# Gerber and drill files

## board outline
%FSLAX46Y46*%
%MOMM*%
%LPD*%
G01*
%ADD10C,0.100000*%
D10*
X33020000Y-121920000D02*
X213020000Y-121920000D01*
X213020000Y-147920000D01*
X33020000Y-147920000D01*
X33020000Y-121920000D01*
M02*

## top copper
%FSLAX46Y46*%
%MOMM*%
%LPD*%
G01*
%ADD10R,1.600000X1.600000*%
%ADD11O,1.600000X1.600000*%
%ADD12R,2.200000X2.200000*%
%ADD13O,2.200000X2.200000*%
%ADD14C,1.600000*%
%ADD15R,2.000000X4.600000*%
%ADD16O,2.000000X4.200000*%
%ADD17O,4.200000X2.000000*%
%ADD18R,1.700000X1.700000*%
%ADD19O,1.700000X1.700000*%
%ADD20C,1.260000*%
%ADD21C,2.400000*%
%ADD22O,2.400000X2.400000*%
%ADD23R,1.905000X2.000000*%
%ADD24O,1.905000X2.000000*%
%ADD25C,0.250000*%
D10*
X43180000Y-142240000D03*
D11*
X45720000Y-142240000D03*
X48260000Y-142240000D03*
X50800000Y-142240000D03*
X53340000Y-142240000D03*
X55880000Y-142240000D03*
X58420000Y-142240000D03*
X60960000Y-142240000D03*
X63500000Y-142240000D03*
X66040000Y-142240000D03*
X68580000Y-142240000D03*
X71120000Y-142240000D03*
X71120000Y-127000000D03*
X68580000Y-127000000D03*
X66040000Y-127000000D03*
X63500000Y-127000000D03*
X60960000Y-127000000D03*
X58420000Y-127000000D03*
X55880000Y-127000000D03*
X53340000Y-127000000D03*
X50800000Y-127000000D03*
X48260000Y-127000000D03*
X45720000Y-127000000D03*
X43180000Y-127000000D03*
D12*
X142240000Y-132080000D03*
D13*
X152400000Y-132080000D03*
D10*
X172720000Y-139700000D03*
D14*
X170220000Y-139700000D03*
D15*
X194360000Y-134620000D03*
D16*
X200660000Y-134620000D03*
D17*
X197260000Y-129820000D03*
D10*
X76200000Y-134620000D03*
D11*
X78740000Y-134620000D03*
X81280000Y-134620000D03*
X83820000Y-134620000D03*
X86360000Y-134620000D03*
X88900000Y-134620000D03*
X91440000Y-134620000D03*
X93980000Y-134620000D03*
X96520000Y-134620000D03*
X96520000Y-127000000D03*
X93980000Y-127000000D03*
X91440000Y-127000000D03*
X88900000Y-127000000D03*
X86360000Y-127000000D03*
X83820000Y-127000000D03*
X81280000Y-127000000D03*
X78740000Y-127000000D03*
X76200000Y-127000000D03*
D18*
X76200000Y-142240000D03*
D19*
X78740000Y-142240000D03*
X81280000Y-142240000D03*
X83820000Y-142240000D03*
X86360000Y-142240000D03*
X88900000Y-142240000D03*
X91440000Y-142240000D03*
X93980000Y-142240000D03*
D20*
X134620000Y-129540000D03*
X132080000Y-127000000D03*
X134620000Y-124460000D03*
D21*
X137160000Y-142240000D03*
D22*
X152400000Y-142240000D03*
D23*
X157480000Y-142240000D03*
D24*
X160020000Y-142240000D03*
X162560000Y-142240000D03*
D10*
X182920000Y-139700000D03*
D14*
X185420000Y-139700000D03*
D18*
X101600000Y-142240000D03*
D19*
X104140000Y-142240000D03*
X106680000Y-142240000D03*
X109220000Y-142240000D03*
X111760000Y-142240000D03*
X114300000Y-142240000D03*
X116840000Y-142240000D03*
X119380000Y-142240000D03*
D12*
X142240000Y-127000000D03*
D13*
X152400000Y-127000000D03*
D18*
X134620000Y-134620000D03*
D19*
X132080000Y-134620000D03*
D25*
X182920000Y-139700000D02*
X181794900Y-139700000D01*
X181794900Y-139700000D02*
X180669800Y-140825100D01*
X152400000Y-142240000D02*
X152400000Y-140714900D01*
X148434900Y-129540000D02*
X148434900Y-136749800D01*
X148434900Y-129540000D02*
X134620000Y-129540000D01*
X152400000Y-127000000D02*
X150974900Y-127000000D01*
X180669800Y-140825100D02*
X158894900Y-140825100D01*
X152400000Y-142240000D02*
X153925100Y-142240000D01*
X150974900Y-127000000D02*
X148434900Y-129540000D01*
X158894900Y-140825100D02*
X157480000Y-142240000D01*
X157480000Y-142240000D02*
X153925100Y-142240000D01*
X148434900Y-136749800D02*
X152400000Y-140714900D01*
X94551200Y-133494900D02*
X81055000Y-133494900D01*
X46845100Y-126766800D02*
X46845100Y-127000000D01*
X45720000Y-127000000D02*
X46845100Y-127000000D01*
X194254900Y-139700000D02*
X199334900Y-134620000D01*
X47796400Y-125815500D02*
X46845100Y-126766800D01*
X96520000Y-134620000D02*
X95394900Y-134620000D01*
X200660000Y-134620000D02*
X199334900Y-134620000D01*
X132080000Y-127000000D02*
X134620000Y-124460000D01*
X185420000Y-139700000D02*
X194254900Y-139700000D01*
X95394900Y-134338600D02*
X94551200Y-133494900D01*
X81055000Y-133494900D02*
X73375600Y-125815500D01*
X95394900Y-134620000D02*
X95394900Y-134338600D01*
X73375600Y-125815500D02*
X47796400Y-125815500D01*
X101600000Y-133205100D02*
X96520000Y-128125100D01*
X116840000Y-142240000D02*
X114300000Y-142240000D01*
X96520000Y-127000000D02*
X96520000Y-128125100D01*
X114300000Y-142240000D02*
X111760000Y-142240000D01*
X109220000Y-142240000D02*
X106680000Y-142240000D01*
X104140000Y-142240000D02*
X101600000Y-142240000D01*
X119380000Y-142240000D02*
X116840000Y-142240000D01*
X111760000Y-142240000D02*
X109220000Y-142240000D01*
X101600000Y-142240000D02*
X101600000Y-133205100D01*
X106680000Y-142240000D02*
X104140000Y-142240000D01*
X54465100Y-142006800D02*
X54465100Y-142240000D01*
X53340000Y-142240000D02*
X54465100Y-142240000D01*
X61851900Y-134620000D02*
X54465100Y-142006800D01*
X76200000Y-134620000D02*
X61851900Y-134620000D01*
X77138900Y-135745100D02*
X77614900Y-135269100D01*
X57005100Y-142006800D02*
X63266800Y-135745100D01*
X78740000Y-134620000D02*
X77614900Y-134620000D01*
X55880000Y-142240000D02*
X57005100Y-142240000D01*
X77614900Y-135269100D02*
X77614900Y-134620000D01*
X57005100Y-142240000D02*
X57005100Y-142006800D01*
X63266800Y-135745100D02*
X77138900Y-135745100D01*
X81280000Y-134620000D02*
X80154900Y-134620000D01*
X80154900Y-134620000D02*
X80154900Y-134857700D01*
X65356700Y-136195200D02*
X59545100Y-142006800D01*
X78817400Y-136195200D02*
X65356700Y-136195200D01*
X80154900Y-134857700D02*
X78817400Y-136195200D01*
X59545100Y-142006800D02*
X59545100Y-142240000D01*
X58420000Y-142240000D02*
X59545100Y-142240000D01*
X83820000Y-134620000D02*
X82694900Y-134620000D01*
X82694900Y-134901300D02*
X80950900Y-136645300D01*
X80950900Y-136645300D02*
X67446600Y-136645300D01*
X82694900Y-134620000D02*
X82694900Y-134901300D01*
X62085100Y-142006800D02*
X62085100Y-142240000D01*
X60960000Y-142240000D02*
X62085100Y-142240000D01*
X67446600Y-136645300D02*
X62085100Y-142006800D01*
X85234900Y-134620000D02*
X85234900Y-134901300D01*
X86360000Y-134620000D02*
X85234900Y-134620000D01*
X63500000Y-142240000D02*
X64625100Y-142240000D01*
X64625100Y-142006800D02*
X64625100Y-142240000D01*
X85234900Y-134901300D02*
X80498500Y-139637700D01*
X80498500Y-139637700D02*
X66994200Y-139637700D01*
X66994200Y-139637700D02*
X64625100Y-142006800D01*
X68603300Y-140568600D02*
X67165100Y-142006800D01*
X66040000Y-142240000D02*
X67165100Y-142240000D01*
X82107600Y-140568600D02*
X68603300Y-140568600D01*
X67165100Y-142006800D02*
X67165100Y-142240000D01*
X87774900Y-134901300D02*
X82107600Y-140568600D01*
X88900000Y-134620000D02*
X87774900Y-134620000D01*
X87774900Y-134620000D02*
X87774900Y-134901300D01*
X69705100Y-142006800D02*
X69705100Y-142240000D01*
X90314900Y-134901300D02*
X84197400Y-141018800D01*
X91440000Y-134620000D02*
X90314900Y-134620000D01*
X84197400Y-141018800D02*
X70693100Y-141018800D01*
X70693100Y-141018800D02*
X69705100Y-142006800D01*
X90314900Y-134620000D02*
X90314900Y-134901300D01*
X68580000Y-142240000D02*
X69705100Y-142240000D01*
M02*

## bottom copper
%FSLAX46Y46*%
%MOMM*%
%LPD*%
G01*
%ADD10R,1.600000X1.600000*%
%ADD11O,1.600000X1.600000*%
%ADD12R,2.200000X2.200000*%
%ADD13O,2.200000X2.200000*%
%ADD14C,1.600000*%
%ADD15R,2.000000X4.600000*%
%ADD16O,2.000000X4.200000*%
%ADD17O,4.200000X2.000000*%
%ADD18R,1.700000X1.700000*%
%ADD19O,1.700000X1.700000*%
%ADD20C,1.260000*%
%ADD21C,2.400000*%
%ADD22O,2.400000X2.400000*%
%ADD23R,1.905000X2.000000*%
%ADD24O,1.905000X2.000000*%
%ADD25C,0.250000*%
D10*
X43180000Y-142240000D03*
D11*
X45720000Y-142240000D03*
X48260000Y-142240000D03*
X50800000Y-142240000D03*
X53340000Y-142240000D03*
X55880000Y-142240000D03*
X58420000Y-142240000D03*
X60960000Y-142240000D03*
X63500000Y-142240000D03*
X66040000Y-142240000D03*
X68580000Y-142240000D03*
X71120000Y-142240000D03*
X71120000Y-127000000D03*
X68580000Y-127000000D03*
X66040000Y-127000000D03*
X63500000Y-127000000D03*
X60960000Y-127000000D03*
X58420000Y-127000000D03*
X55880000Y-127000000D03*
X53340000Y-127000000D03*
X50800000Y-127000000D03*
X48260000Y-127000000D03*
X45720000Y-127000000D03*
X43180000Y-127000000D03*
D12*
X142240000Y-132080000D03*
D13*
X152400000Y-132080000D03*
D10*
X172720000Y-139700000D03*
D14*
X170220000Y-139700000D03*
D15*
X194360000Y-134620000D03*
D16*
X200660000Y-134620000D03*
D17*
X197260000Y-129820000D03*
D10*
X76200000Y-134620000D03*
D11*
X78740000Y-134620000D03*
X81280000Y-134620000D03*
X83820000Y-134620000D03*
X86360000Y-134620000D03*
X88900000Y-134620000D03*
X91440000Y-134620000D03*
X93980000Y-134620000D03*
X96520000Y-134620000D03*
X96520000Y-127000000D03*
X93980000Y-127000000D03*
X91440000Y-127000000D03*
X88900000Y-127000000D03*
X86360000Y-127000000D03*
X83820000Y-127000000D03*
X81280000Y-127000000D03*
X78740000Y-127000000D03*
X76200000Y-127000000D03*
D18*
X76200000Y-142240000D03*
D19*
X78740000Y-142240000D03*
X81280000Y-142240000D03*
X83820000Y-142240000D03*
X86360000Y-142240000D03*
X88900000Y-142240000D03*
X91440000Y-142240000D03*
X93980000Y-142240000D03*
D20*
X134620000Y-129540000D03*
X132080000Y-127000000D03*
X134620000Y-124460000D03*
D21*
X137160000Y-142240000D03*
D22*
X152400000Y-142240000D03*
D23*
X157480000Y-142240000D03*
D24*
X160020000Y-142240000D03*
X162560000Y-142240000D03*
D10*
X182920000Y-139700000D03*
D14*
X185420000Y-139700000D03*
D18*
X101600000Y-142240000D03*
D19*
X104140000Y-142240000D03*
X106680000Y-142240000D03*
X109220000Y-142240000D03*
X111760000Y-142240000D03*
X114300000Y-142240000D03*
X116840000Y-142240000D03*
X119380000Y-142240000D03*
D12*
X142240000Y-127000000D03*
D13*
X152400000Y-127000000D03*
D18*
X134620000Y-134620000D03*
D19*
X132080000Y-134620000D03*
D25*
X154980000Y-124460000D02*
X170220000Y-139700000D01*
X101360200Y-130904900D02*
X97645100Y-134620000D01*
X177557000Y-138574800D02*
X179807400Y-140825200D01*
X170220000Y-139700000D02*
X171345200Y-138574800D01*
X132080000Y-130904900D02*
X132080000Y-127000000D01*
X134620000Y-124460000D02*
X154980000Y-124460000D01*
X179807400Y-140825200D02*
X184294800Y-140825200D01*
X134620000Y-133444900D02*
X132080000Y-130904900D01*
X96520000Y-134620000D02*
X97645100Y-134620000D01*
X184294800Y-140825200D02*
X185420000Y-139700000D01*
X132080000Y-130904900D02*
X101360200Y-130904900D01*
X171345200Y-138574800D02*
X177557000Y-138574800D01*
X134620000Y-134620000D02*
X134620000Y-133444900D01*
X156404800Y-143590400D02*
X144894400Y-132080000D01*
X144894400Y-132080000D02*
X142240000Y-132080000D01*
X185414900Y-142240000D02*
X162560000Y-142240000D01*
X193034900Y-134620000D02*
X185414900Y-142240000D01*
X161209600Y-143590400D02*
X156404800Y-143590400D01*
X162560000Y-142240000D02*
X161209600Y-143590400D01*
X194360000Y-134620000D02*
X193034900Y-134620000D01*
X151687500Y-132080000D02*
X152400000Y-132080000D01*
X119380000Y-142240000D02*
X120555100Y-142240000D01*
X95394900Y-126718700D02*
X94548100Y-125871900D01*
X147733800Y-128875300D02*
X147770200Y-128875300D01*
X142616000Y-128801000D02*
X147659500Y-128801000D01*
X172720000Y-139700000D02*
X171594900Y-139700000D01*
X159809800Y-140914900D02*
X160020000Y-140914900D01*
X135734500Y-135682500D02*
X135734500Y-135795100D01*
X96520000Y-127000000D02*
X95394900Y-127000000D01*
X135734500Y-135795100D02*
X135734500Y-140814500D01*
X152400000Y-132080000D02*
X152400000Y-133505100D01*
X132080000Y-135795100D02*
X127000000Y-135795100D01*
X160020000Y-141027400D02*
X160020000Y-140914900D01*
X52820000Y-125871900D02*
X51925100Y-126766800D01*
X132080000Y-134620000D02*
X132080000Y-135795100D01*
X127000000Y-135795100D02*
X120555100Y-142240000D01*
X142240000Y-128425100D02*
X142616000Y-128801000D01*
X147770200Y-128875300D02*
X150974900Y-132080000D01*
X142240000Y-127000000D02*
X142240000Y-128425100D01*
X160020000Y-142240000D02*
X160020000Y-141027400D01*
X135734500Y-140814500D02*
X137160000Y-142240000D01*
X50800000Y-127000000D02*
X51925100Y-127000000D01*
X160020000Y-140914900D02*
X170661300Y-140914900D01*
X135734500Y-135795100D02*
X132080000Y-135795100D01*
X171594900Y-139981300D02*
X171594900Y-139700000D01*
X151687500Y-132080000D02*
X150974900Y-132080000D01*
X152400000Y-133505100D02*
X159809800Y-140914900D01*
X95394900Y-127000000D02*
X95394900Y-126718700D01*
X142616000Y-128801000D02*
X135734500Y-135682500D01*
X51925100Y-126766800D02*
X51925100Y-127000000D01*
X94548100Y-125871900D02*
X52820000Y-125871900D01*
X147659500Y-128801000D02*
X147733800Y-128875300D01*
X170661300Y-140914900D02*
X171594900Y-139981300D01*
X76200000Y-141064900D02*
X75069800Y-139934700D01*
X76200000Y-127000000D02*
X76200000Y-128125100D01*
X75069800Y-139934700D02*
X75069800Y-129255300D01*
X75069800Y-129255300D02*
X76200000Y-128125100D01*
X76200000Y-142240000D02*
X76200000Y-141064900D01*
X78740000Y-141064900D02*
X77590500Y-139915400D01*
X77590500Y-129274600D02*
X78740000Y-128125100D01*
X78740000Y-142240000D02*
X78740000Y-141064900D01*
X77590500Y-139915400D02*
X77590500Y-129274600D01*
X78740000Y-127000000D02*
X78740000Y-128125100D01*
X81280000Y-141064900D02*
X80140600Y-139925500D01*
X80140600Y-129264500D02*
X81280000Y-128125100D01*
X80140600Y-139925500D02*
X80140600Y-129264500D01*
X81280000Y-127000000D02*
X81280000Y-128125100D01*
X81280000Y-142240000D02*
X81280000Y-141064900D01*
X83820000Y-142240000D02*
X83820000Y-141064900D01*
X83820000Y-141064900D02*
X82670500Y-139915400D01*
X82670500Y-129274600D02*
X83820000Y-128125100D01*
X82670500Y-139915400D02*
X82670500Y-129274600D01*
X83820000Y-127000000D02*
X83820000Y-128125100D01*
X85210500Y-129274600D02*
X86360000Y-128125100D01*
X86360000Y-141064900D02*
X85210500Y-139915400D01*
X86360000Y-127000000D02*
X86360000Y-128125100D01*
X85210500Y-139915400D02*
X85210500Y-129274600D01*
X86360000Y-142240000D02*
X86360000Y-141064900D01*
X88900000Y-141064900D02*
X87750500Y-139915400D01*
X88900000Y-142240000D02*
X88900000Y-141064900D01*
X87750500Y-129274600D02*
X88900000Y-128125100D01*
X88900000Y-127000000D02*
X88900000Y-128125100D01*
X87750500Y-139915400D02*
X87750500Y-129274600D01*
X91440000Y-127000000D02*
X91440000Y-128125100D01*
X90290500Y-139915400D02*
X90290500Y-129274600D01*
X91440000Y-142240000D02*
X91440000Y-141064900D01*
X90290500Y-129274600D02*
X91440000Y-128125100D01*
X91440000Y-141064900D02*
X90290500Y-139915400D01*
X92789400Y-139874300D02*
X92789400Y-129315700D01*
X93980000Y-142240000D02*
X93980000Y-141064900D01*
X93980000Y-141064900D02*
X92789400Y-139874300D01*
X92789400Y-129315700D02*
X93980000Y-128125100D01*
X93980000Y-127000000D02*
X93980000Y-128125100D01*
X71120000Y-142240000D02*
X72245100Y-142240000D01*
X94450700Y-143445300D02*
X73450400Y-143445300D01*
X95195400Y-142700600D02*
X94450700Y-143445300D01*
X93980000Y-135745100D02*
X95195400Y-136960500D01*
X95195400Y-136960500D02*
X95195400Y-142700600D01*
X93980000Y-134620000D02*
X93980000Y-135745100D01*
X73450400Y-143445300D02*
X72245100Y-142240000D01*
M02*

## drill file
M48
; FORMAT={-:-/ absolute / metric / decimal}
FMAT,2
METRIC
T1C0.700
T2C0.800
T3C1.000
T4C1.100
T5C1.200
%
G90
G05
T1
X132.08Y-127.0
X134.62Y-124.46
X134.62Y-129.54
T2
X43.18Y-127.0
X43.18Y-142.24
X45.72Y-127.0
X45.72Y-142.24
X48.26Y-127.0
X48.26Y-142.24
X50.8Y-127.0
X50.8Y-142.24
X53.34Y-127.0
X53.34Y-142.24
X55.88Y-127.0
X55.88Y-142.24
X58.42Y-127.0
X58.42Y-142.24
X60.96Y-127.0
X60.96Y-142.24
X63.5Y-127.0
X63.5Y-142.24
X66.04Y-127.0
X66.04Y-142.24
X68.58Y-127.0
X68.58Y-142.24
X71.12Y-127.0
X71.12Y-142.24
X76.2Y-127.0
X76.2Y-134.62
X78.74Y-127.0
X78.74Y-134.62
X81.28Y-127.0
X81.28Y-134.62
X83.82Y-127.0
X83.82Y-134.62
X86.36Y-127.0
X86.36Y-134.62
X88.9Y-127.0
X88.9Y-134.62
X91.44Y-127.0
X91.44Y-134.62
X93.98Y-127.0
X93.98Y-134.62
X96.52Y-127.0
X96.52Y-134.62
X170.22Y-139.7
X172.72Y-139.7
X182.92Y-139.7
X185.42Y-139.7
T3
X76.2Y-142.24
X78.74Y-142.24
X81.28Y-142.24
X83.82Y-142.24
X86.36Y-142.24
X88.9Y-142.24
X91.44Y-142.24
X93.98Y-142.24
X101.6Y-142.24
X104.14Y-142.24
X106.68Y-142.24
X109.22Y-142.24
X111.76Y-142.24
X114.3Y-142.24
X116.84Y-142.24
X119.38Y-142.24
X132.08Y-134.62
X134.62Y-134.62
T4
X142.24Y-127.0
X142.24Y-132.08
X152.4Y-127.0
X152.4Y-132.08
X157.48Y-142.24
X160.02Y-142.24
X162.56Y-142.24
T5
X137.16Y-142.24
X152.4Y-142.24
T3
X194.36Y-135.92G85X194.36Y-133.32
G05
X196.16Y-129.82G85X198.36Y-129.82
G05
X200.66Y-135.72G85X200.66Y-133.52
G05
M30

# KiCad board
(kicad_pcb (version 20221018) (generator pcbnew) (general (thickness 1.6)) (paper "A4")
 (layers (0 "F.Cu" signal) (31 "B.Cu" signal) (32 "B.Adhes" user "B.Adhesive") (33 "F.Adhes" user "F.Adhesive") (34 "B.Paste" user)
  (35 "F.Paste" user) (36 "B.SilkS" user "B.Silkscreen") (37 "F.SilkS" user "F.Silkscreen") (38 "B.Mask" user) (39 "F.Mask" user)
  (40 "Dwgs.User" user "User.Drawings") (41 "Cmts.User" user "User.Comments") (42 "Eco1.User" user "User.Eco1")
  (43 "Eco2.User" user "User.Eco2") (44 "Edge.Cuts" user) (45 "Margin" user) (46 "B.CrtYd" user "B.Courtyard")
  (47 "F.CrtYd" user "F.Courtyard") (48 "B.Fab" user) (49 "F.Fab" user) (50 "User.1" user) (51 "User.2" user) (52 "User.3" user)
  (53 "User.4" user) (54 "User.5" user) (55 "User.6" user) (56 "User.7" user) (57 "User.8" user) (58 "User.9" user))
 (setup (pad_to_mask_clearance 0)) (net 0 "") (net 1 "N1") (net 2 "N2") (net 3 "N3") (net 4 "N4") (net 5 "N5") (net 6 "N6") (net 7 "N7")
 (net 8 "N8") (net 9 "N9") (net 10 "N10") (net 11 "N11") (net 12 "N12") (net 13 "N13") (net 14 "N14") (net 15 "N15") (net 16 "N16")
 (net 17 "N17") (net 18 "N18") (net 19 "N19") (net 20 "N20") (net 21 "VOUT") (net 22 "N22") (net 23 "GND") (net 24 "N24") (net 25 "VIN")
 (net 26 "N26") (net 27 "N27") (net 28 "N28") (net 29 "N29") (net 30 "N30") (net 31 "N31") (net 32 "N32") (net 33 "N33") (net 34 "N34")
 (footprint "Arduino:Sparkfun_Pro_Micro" (layer "F.Cu") (at 71.12 127 -90)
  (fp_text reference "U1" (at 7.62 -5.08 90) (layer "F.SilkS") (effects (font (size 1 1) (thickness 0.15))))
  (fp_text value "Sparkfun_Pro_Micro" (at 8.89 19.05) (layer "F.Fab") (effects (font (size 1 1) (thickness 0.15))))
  (pad "1" thru_hole rect (at 15.24 27.94 270) (size 1.6 1.6) (drill 0.8) (layers "*.Cu" "*.Mask") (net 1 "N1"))
  (pad "2" thru_hole oval (at 15.24 25.4 270) (size 1.6 1.6) (drill 0.8) (layers "*.Cu" "*.Mask") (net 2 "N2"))
  (pad "3" thru_hole oval (at 15.24 22.86 270) (size 1.6 1.6) (drill 0.8) (layers "*.Cu" "*.Mask") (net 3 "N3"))
  (pad "4" thru_hole oval (at 15.24 20.32 270) (size 1.6 1.6) (drill 0.8) (layers "*.Cu" "*.Mask") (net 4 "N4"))
  (pad "5" thru_hole oval (at 15.24 17.78 270) (size 1.6 1.6) (drill 0.8) (layers "*.Cu" "*.Mask") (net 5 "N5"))
  (pad "6" thru_hole oval (at 15.24 15.24 270) (size 1.6 1.6) (drill 0.8) (layers "*.Cu" "*.Mask") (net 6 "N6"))
  (pad "7" thru_hole oval (at 15.24 12.7 270) (size 1.6 1.6) (drill 0.8) (layers "*.Cu" "*.Mask") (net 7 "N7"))
  (pad "8" thru_hole oval (at 15.24 10.16 270) (size 1.6 1.6) (drill 0.8) (layers "*.Cu" "*.Mask") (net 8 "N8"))
  (pad "9" thru_hole oval (at 15.24 7.62 270) (size 1.6 1.6) (drill 0.8) (layers "*.Cu" "*.Mask") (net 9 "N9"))
  (pad "10" thru_hole oval (at 15.24 5.08 270) (size 1.6 1.6) (drill 0.8) (layers "*.Cu" "*.Mask") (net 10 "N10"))
  (pad "11" thru_hole oval (at 15.24 2.54 270) (size 1.6 1.6) (drill 0.8) (layers "*.Cu" "*.Mask") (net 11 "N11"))
  (pad "12" thru_hole oval (at 15.24 0 270) (size 1.6 1.6) (drill 0.8) (layers "*.Cu" "*.Mask") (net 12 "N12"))
  (pad "13" thru_hole oval (at 0 0 270) (size 1.6 1.6) (drill 0.8) (layers "*.Cu" "*.Mask") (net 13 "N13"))
  (pad "14" thru_hole oval (at 0 2.54 270) (size 1.6 1.6) (drill 0.8) (layers "*.Cu" "*.Mask") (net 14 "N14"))
  (pad "15" thru_hole oval (at 0 5.08 270) (size 1.6 1.6) (drill 0.8) (layers "*.Cu" "*.Mask") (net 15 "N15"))
  (pad "16" thru_hole oval (at 0 7.62 270) (size 1.6 1.6) (drill 0.8) (layers "*.Cu" "*.Mask") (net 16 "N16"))
  (pad "17" thru_hole oval (at 0 10.16 270) (size 1.6 1.6) (drill 0.8) (layers "*.Cu" "*.Mask") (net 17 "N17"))
  (pad "18" thru_hole oval (at 0 12.7 270) (size 1.6 1.6) (drill 0.8) (layers "*.Cu" "*.Mask") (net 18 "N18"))
  (pad "19" thru_hole oval (at 0 15.24 270) (size 1.6 1.6) (drill 0.8) (layers "*.Cu" "*.Mask") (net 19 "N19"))
  (pad "20" thru_hole oval (at 0 17.78 270) (size 1.6 1.6) (drill 0.8) (layers "*.Cu" "*.Mask") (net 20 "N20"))
  (pad "21" thru_hole oval (at 0 20.32 270) (size 1.6 1.6) (drill 0.8) (layers "*.Cu" "*.Mask") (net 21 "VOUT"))
  (pad "22" thru_hole oval (at 0 22.86 270) (size 1.6 1.6) (drill 0.8) (layers "*.Cu" "*.Mask") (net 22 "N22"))
  (pad "23" thru_hole oval (at 0 25.4 270) (size 1.6 1.6) (drill 0.8) (layers "*.Cu" "*.Mask") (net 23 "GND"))
  (pad "24" thru_hole oval (at 0 27.94 270) (size 1.6 1.6) (drill 0.8) (layers "*.Cu" "*.Mask") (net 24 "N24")))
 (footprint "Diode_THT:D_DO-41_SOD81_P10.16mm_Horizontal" (layer "F.Cu") (at 142.24 132.08)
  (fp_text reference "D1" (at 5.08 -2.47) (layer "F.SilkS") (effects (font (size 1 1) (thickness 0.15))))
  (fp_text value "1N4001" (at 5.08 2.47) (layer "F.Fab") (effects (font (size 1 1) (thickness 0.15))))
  (pad "1" thru_hole rect (at 0 0) (size 2.2 2.2) (drill 1.1) (layers "*.Cu" "*.Mask") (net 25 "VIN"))
  (pad "2" thru_hole oval (at 10.16 0) (size 2.2 2.2) (drill 1.1) (layers "*.Cu" "*.Mask") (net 21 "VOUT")))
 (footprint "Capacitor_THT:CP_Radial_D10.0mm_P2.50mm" (layer "F.Cu") (at 172.72 139.7 180)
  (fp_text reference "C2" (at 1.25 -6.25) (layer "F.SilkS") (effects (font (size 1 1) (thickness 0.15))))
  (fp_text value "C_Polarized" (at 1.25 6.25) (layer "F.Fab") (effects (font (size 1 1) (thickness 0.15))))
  (pad "1" thru_hole rect (at 0 0 180) (size 1.6 1.6) (drill 0.8) (layers "*.Cu" "*.Mask") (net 21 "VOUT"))
  (pad "2" thru_hole circle (at 2.5 0 180) (size 1.6 1.6) (drill 0.8) (layers "*.Cu" "*.Mask") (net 23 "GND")))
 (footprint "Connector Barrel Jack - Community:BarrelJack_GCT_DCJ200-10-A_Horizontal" (layer "F.Cu") (at 194.36 134.62 90)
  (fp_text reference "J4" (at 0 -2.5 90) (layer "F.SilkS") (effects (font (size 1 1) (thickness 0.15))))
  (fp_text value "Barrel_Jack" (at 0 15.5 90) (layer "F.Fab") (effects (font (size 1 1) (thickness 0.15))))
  (pad "1" thru_hole rect (at 0 0 90) (size 4.6 2) (drill oval 3.6 1) (layers "*.Cu" "*.Mask") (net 25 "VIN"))
  (pad "2" thru_hole oval (at 0 6.3 90) (size 4.2 2) (drill oval 3.2 1) (layers "*.Cu" "*.Mask") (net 23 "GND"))
  (pad "3" thru_hole oval (at 4.8 2.9 90) (size 2 4.2) (drill oval 1 3.2) (layers "*.Cu" "*.Mask")))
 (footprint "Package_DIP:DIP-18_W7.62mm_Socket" (layer "F.Cu") (at 76.2 134.62 90)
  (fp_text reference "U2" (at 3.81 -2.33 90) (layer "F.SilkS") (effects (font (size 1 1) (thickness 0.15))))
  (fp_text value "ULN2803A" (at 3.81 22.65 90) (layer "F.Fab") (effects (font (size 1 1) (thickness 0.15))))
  (pad "1" thru_hole rect (at 0 0 90) (size 1.6 1.6) (drill 0.8) (layers "*.Cu" "*.Mask") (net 5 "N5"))
  (pad "2" thru_hole oval (at 0 2.54 90) (size 1.6 1.6) (drill 0.8) (layers "*.Cu" "*.Mask") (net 6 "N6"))
  (pad "3" thru_hole oval (at 0 5.08 90) (size 1.6 1.6) (drill 0.8) (layers "*.Cu" "*.Mask") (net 7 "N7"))
  (pad "4" thru_hole oval (at 0 7.62 90) (size 1.6 1.6) (drill 0.8) (layers "*.Cu" "*.Mask") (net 8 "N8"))
  (pad "5" thru_hole oval (at 0 10.16 90) (size 1.6 1.6) (drill 0.8) (layers "*.Cu" "*.Mask") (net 9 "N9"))
  (pad "6" thru_hole oval (at 0 12.7 90) (size 1.6 1.6) (drill 0.8) (layers "*.Cu" "*.Mask") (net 10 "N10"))
  (pad "7" thru_hole oval (at 0 15.24 90) (size 1.6 1.6) (drill 0.8) (layers "*.Cu" "*.Mask") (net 11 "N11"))
  (pad "8" thru_hole oval (at 0 17.78 90) (size 1.6 1.6) (drill 0.8) (layers "*.Cu" "*.Mask") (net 12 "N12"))
  (pad "9" thru_hole oval (at 0 20.32 90) (size 1.6 1.6) (drill 0.8) (layers "*.Cu" "*.Mask") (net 23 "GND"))
  (pad "10" thru_hole oval (at 7.62 20.32 90) (size 1.6 1.6) (drill 0.8) (layers "*.Cu" "*.Mask") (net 21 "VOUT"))
  (pad "11" thru_hole oval (at 7.62 17.78 90) (size 1.6 1.6) (drill 0.8) (layers "*.Cu" "*.Mask") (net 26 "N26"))
  (pad "12" thru_hole oval (at 7.62 15.24 90) (size 1.6 1.6) (drill 0.8) (layers "*.Cu" "*.Mask") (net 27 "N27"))
  (pad "13" thru_hole oval (at 7.62 12.7 90) (size 1.6 1.6) (drill 0.8) (layers "*.Cu" "*.Mask") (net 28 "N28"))
  (pad "14" thru_hole oval (at 7.62 10.16 90) (size 1.6 1.6) (drill 0.8) (layers "*.Cu" "*.Mask") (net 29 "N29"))
  (pad "15" thru_hole oval (at 7.62 7.62 90) (size 1.6 1.6) (drill 0.8) (layers "*.Cu" "*.Mask") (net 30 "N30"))
  (pad "16" thru_hole oval (at 7.62 5.08 90) (size 1.6 1.6) (drill 0.8) (layers "*.Cu" "*.Mask") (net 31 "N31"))
  (pad "17" thru_hole oval (at 7.62 2.54 90) (size 1.6 1.6) (drill 0.8) (layers "*.Cu" "*.Mask") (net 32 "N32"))
  (pad "18" thru_hole oval (at 7.62 0 90) (size 1.6 1.6) (drill 0.8) (layers "*.Cu" "*.Mask") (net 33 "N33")))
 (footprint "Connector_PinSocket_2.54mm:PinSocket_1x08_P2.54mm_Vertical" (layer "F.Cu") (at 76.2 142.24 90)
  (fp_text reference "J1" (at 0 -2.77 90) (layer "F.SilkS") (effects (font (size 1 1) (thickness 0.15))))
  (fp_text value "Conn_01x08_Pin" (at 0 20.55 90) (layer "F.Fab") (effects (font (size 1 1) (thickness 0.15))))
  (pad "1" thru_hole rect (at 0 0 90) (size 1.7 1.7) (drill 1) (layers "*.Cu" "*.Mask") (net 33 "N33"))
  (pad "2" thru_hole oval (at 0 2.54 90) (size 1.7 1.7) (drill 1) (layers "*.Cu" "*.Mask") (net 32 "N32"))
  (pad "3" thru_hole oval (at 0 5.08 90) (size 1.7 1.7) (drill 1) (layers "*.Cu" "*.Mask") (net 31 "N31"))
  (pad "4" thru_hole oval (at 0 7.62 90) (size 1.7 1.7) (drill 1) (layers "*.Cu" "*.Mask") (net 30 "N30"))
  (pad "5" thru_hole oval (at 0 10.16 90) (size 1.7 1.7) (drill 1) (layers "*.Cu" "*.Mask") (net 29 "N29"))
  (pad "6" thru_hole oval (at 0 12.7 90) (size 1.7 1.7) (drill 1) (layers "*.Cu" "*.Mask") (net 28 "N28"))
  (pad "7" thru_hole oval (at 0 15.24 90) (size 1.7 1.7) (drill 1) (layers "*.Cu" "*.Mask") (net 27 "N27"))
  (pad "8" thru_hole oval (at 0 17.78 90) (size 1.7 1.7) (drill 1) (layers "*.Cu" "*.Mask") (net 26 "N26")))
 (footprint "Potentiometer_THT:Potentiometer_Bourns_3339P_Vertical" (layer "F.Cu") (at 134.62 129.54)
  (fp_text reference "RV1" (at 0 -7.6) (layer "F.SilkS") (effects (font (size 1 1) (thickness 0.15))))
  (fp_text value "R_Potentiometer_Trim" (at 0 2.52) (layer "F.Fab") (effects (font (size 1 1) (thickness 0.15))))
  (pad "1" thru_hole circle (at 0 0) (size 1.26 1.26) (drill 0.7) (layers "*.Cu" "*.Mask") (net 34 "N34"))
  (pad "2" thru_hole circle (at -2.54 -2.54) (size 1.26 1.26) (drill 0.7) (layers "*.Cu" "*.Mask") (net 23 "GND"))
  (pad "3" thru_hole circle (at 0 -5.08) (size 1.26 1.26) (drill 0.7) (layers "*.Cu" "*.Mask") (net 23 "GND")))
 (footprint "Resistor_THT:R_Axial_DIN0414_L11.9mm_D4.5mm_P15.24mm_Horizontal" (layer "F.Cu") (at 137.16 142.24)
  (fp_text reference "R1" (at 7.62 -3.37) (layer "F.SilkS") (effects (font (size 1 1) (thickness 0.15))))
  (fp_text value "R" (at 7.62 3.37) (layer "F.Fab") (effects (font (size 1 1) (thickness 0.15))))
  (pad "1" thru_hole circle (at 0 0) (size 2.4 2.4) (drill 1.2) (layers "*.Cu" "*.Mask") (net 21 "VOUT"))
  (pad "2" thru_hole oval (at 15.24 0) (size 2.4 2.4) (drill 1.2) (layers "*.Cu" "*.Mask") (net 34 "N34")))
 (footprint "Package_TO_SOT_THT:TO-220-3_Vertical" (layer "F.Cu") (at 157.48 142.24)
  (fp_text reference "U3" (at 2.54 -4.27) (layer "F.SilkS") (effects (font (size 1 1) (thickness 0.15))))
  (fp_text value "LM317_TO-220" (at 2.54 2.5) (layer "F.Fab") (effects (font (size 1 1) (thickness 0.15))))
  (pad "1" thru_hole rect (at 0 0) (size 1.905 2) (drill 1.1) (layers "*.Cu" "*.Mask") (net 34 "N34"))
  (pad "2" thru_hole oval (at 2.54 0) (size 1.905 2) (drill 1.1) (layers "*.Cu" "*.Mask") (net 21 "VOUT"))
  (pad "3" thru_hole oval (at 5.08 0) (size 1.905 2) (drill 1.1) (layers "*.Cu" "*.Mask") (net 25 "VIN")))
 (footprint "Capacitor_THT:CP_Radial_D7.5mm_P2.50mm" (layer "F.Cu") (at 182.92 139.7)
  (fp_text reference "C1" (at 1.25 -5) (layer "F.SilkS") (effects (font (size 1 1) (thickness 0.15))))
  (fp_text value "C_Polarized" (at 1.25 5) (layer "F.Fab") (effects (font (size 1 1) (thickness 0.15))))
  (pad "1" thru_hole rect (at 0 0) (size 1.6 1.6) (drill 0.8) (layers "*.Cu" "*.Mask") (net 34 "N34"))
  (pad "2" thru_hole circle (at 2.5 0) (size 1.6 1.6) (drill 0.8) (layers "*.Cu" "*.Mask") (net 23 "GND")))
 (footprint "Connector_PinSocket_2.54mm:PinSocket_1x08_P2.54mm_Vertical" (layer "F.Cu") (at 101.6 142.24 90)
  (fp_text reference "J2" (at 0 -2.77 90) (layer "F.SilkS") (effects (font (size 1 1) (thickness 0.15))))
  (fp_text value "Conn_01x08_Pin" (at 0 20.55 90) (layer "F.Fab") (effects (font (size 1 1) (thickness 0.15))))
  (pad "1" thru_hole rect (at 0 0 90) (size 1.7 1.7) (drill 1) (layers "*.Cu" "*.Mask") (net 21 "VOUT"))
  (pad "2" thru_hole oval (at 0 2.54 90) (size 1.7 1.7) (drill 1) (layers "*.Cu" "*.Mask") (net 21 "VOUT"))
  (pad "3" thru_hole oval (at 0 5.08 90) (size 1.7 1.7) (drill 1) (layers "*.Cu" "*.Mask") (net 21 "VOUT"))
  (pad "4" thru_hole oval (at 0 7.62 90) (size 1.7 1.7) (drill 1) (layers "*.Cu" "*.Mask") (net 21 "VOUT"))
  (pad "5" thru_hole oval (at 0 10.16 90) (size 1.7 1.7) (drill 1) (layers "*.Cu" "*.Mask") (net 21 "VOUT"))
  (pad "6" thru_hole oval (at 0 12.7 90) (size 1.7 1.7) (drill 1) (layers "*.Cu" "*.Mask") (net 21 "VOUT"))
  (pad "7" thru_hole oval (at 0 15.24 90) (size 1.7 1.7) (drill 1) (layers "*.Cu" "*.Mask") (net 21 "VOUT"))
  (pad "8" thru_hole oval (at 0 17.78 90) (size 1.7 1.7) (drill 1) (layers "*.Cu" "*.Mask") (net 21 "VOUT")))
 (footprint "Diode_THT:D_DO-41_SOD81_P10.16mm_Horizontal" (layer "F.Cu") (at 142.24 127)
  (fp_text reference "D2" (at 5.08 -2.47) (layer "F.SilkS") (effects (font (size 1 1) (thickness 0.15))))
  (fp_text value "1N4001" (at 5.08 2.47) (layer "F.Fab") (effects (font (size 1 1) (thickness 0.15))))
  (pad "1" thru_hole rect (at 0 0) (size 2.2 2.2) (drill 1.1) (layers "*.Cu" "*.Mask") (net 21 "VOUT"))
  (pad "2" thru_hole oval (at 10.16 0) (size 2.2 2.2) (drill 1.1) (layers "*.Cu" "*.Mask") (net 34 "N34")))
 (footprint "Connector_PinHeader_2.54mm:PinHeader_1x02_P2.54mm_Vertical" (layer "F.Cu") (at 134.62 134.62 -90)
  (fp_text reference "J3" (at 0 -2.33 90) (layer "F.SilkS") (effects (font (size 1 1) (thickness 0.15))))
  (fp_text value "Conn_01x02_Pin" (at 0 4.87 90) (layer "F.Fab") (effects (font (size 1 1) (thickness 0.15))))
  (pad "1" thru_hole rect (at 0 0 270) (size 1.7 1.7) (drill 1) (layers "*.Cu" "*.Mask") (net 23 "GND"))
  (pad "2" thru_hole oval (at 0 2.54 270) (size 1.7 1.7) (drill 1) (layers "*.Cu" "*.Mask") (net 21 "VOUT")))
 (gr_rect (start 33.02 121.92) (end 213.02 147.92) (stroke (width 0.1) (type default)) (fill none) (layer "Edge.Cuts"))
 (segment (start 182.92 139.7) (end 181.7949 139.7) (width 0.25) (layer "F.Cu") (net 34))
 (segment (start 181.7949 139.7) (end 180.6698 140.8251) (width 0.25) (layer "F.Cu") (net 34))
 (segment (start 152.4 142.24) (end 152.4 140.7149) (width 0.25) (layer "F.Cu") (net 34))
 (segment (start 148.4349 129.54) (end 148.4349 136.7498) (width 0.25) (layer "F.Cu") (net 34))
 (segment (start 148.4349 129.54) (end 134.62 129.54) (width 0.25) (layer "F.Cu") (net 34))
 (segment (start 152.4 127) (end 150.9749 127) (width 0.25) (layer "F.Cu") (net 34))
 (segment (start 180.6698 140.8251) (end 158.8949 140.8251) (width 0.25) (layer "F.Cu") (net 34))
 (segment (start 152.4 142.24) (end 153.9251 142.24) (width 0.25) (layer "F.Cu") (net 34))
 (segment (start 150.9749 127) (end 148.4349 129.54) (width 0.25) (layer "F.Cu") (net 34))
 (segment (start 158.8949 140.8251) (end 157.48 142.24) (width 0.25) (layer "F.Cu") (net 34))
 (segment (start 157.48 142.24) (end 153.9251 142.24) (width 0.25) (layer "F.Cu") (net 34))
 (segment (start 148.4349 136.7498) (end 152.4 140.7149) (width 0.25) (layer "F.Cu") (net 34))
 (segment (start 94.5512 133.4949) (end 81.055 133.4949) (width 0.25) (layer "F.Cu") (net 23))
 (segment (start 46.8451 126.7668) (end 46.8451 127) (width 0.25) (layer "F.Cu") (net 23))
 (segment (start 45.72 127) (end 46.8451 127) (width 0.25) (layer "F.Cu") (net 23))
 (segment (start 194.2549 139.7) (end 199.3349 134.62) (width 0.25) (layer "F.Cu") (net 23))
 (segment (start 47.7964 125.8155) (end 46.8451 126.7668) (width 0.25) (layer "F.Cu") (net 23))
 (segment (start 96.52 134.62) (end 95.3949 134.62) (width 0.25) (layer "F.Cu") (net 23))
 (segment (start 200.66 134.62) (end 199.3349 134.62) (width 0.25) (layer "F.Cu") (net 23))
 (segment (start 132.08 127) (end 134.62 124.46) (width 0.25) (layer "F.Cu") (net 23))
 (segment (start 185.42 139.7) (end 194.2549 139.7) (width 0.25) (layer "F.Cu") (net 23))
 (segment (start 95.3949 134.3386) (end 94.5512 133.4949) (width 0.25) (layer "F.Cu") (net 23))
 (segment (start 81.055 133.4949) (end 73.3756 125.8155) (width 0.25) (layer "F.Cu") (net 23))
 (segment (start 95.3949 134.62) (end 95.3949 134.3386) (width 0.25) (layer "F.Cu") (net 23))
 (segment (start 73.3756 125.8155) (end 47.7964 125.8155) (width 0.25) (layer "F.Cu") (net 23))
 (segment (start 154.98 124.46) (end 170.22 139.7) (width 0.25) (layer "B.Cu") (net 23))
 (segment (start 101.3602 130.9049) (end 97.6451 134.62) (width 0.25) (layer "B.Cu") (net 23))
 (segment (start 177.557 138.5748) (end 179.8074 140.8252) (width 0.25) (layer "B.Cu") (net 23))
 (segment (start 170.22 139.7) (end 171.3452 138.5748) (width 0.25) (layer "B.Cu") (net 23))
 (segment (start 132.08 130.9049) (end 132.08 127) (width 0.25) (layer "B.Cu") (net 23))
 (segment (start 134.62 124.46) (end 154.98 124.46) (width 0.25) (layer "B.Cu") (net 23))
 (segment (start 179.8074 140.8252) (end 184.2948 140.8252) (width 0.25) (layer "B.Cu") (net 23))
 (segment (start 134.62 133.4449) (end 132.08 130.9049) (width 0.25) (layer "B.Cu") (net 23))
 (segment (start 96.52 134.62) (end 97.6451 134.62) (width 0.25) (layer "B.Cu") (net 23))
 (segment (start 184.2948 140.8252) (end 185.42 139.7) (width 0.25) (layer "B.Cu") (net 23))
 (segment (start 132.08 130.9049) (end 101.3602 130.9049) (width 0.25) (layer "B.Cu") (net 23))
 (segment (start 171.3452 138.5748) (end 177.557 138.5748) (width 0.25) (layer "B.Cu") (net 23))
 (segment (start 134.62 134.62) (end 134.62 133.4449) (width 0.25) (layer "B.Cu") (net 23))
 (segment (start 156.4048 143.5904) (end 144.8944 132.08) (width 0.25) (layer "B.Cu") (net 25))
 (segment (start 144.8944 132.08) (end 142.24 132.08) (width 0.25) (layer "B.Cu") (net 25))
 (segment (start 185.4149 142.24) (end 162.56 142.24) (width 0.25) (layer "B.Cu") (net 25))
 (segment (start 193.0349 134.62) (end 185.4149 142.24) (width 0.25) (layer "B.Cu") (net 25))
 (segment (start 161.2096 143.5904) (end 156.4048 143.5904) (width 0.25) (layer "B.Cu") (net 25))
 (segment (start 162.56 142.24) (end 161.2096 143.5904) (width 0.25) (layer "B.Cu") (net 25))
 (segment (start 194.36 134.62) (end 193.0349 134.62) (width 0.25) (layer "B.Cu") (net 25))
 (segment (start 101.6 133.2051) (end 96.52 128.1251) (width 0.25) (layer "F.Cu") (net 21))
 (segment (start 116.84 142.24) (end 114.3 142.24) (width 0.25) (layer "F.Cu") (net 21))
 (segment (start 96.52 127) (end 96.52 128.1251) (width 0.25) (layer "F.Cu") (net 21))
 (segment (start 114.3 142.24) (end 111.76 142.24) (width 0.25) (layer "F.Cu") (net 21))
 (segment (start 109.22 142.24) (end 106.68 142.24) (width 0.25) (layer "F.Cu") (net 21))
 (segment (start 104.14 142.24) (end 101.6 142.24) (width 0.25) (layer "F.Cu") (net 21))
 (segment (start 119.38 142.24) (end 116.84 142.24) (width 0.25) (layer "F.Cu") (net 21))
 (segment (start 111.76 142.24) (end 109.22 142.24) (width 0.25) (layer "F.Cu") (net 21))
 (segment (start 101.6 142.24) (end 101.6 133.2051) (width 0.25) (layer "F.Cu") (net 21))
 (segment (start 106.68 142.24) (end 104.14 142.24) (width 0.25) (layer "F.Cu") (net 21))
 (segment (start 151.6875 132.08) (end 152.4 132.08) (width 0.25) (layer "B.Cu") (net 21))
 (segment (start 119.38 142.24) (end 120.5551 142.24) (width 0.25) (layer "B.Cu") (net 21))
 (segment (start 95.3949 126.7187) (end 94.5481 125.8719) (width 0.25) (layer "B.Cu") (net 21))
 (segment (start 147.7338 128.8753) (end 147.7702 128.8753) (width 0.25) (layer "B.Cu") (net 21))
 (segment (start 142.616 128.801) (end 147.6595 128.801) (width 0.25) (layer "B.Cu") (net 21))
 (segment (start 172.72 139.7) (end 171.5949 139.7) (width 0.25) (layer "B.Cu") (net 21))
 (segment (start 159.8098 140.9149) (end 160.02 140.9149) (width 0.25) (layer "B.Cu") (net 21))
 (segment (start 135.7345 135.6825) (end 135.7345 135.7951) (width 0.25) (layer "B.Cu") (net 21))
 (segment (start 96.52 127) (end 95.3949 127) (width 0.25) (layer "B.Cu") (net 21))
 (segment (start 135.7345 135.7951) (end 135.7345 140.8145) (width 0.25) (layer "B.Cu") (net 21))
 (segment (start 152.4 132.08) (end 152.4 133.5051) (width 0.25) (layer "B.Cu") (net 21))
 (segment (start 132.08 135.7951) (end 127 135.7951) (width 0.25) (layer "B.Cu") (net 21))
 (segment (start 160.02 141.0274) (end 160.02 140.9149) (width 0.25) (layer "B.Cu") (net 21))
 (segment (start 52.82 125.8719) (end 51.9251 126.7668) (width 0.25) (layer "B.Cu") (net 21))
 (segment (start 132.08 134.62) (end 132.08 135.7951) (width 0.25) (layer "B.Cu") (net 21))
 (segment (start 127 135.7951) (end 120.5551 142.24) (width 0.25) (layer "B.Cu") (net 21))
 (segment (start 142.24 128.4251) (end 142.616 128.801) (width 0.25) (layer "B.Cu") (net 21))
 (segment (start 147.7702 128.8753) (end 150.9749 132.08) (width 0.25) (layer "B.Cu") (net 21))
 (segment (start 142.24 127) (end 142.24 128.4251) (width 0.25) (layer "B.Cu") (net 21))
 (segment (start 160.02 142.24) (end 160.02 141.0274) (width 0.25) (layer "B.Cu") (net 21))
 (segment (start 135.7345 140.8145) (end 137.16 142.24) (width 0.25) (layer "B.Cu") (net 21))
 (segment (start 50.8 127) (end 51.9251 127) (width 0.25) (layer "B.Cu") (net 21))
 (segment (start 160.02 140.9149) (end 170.6613 140.9149) (width 0.25) (layer "B.Cu") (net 21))
 (segment (start 135.7345 135.7951) (end 132.08 135.7951) (width 0.25) (layer "B.Cu") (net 21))
 (segment (start 171.5949 139.9813) (end 171.5949 139.7) (width 0.25) (layer "B.Cu") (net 21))
 (segment (start 151.6875 132.08) (end 150.9749 132.08) (width 0.25) (layer "B.Cu") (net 21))
 (segment (start 152.4 133.5051) (end 159.8098 140.9149) (width 0.25) (layer "B.Cu") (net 21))
 (segment (start 95.3949 127) (end 95.3949 126.7187) (width 0.25) (layer "B.Cu") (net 21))
 (segment (start 142.616 128.801) (end 135.7345 135.6825) (width 0.25) (layer "B.Cu") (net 21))
 (segment (start 51.9251 126.7668) (end 51.9251 127) (width 0.25) (layer "B.Cu") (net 21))
 (segment (start 94.5481 125.8719) (end 52.82 125.8719) (width 0.25) (layer "B.Cu") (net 21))
 (segment (start 147.6595 128.801) (end 147.7338 128.8753) (width 0.25) (layer "B.Cu") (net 21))
 (segment (start 170.6613 140.9149) (end 171.5949 139.9813) (width 0.25) (layer "B.Cu") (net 21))
 (segment (start 76.2 141.0649) (end 75.0698 139.9347) (width 0.25) (layer "B.Cu") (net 33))
 (segment (start 76.2 127) (end 76.2 128.1251) (width 0.25) (layer "B.Cu") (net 33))
 (segment (start 75.0698 139.9347) (end 75.0698 129.2553) (width 0.25) (layer "B.Cu") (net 33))
 (segment (start 75.0698 129.2553) (end 76.2 128.1251) (width 0.25) (layer "B.Cu") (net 33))
 (segment (start 76.2 142.24) (end 76.2 141.0649) (width 0.25) (layer "B.Cu") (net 33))
 (segment (start 78.74 141.0649) (end 77.5905 139.9154) (width 0.25) (layer "B.Cu") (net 32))
 (segment (start 77.5905 129.2746) (end 78.74 128.1251) (width 0.25) (layer "B.Cu") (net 32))
 (segment (start 78.74 142.24) (end 78.74 141.0649) (width 0.25) (layer "B.Cu") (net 32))
 (segment (start 77.5905 139.9154) (end 77.5905 129.2746) (width 0.25) (layer "B.Cu") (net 32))
 (segment (start 78.74 127) (end 78.74 128.1251) (width 0.25) (layer "B.Cu") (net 32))
 (segment (start 81.28 141.0649) (end 80.1406 139.9255) (width 0.25) (layer "B.Cu") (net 31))
 (segment (start 80.1406 129.2645) (end 81.28 128.1251) (width 0.25) (layer "B.Cu") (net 31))
 (segment (start 80.1406 139.9255) (end 80.1406 129.2645) (width 0.25) (layer "B.Cu") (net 31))
 (segment (start 81.28 127) (end 81.28 128.1251) (width 0.25) (layer "B.Cu") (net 31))
 (segment (start 81.28 142.24) (end 81.28 141.0649) (width 0.25) (layer "B.Cu") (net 31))
 (segment (start 83.82 142.24) (end 83.82 141.0649) (width 0.25) (layer "B.Cu") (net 30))
 (segment (start 83.82 141.0649) (end 82.6705 139.9154) (width 0.25) (layer "B.Cu") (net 30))
 (segment (start 82.6705 129.2746) (end 83.82 128.1251) (width 0.25) (layer "B.Cu") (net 30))
 (segment (start 82.6705 139.9154) (end 82.6705 129.2746) (width 0.25) (layer "B.Cu") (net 30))
 (segment (start 83.82 127) (end 83.82 128.1251) (width 0.25) (layer "B.Cu") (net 30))
 (segment (start 85.2105 129.2746) (end 86.36 128.1251) (width 0.25) (layer "B.Cu") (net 29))
 (segment (start 86.36 141.0649) (end 85.2105 139.9154) (width 0.25) (layer "B.Cu") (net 29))
 (segment (start 86.36 127) (end 86.36 128.1251) (width 0.25) (layer "B.Cu") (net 29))
 (segment (start 85.2105 139.9154) (end 85.2105 129.2746) (width 0.25) (layer "B.Cu") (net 29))
 (segment (start 86.36 142.24) (end 86.36 141.0649) (width 0.25) (layer "B.Cu") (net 29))
 (segment (start 88.9 141.0649) (end 87.7505 139.9154) (width 0.25) (layer "B.Cu") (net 28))
 (segment (start 88.9 142.24) (end 88.9 141.0649) (width 0.25) (layer "B.Cu") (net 28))
 (segment (start 87.7505 129.2746) (end 88.9 128.1251) (width 0.25) (layer "B.Cu") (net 28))
 (segment (start 88.9 127) (end 88.9 128.1251) (width 0.25) (layer "B.Cu") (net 28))
 (segment (start 87.7505 139.9154) (end 87.7505 129.2746) (width 0.25) (layer "B.Cu") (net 28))
 (segment (start 91.44 127) (end 91.44 128.1251) (width 0.25) (layer "B.Cu") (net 27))
 (segment (start 90.2905 139.9154) (end 90.2905 129.2746) (width 0.25) (layer "B.Cu") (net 27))
 (segment (start 91.44 142.24) (end 91.44 141.0649) (width 0.25) (layer "B.Cu") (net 27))
 (segment (start 90.2905 129.2746) (end 91.44 128.1251) (width 0.25) (layer "B.Cu") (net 27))
 (segment (start 91.44 141.0649) (end 90.2905 139.9154) (width 0.25) (layer "B.Cu") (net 27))
 (segment (start 92.7894 139.8743) (end 92.7894 129.3157) (width 0.25) (layer "B.Cu") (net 26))
 (segment (start 93.98 142.24) (end 93.98 141.0649) (width 0.25) (layer "B.Cu") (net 26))
 (segment (start 93.98 141.0649) (end 92.7894 139.8743) (width 0.25) (layer "B.Cu") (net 26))
 (segment (start 92.7894 129.3157) (end 93.98 128.1251) (width 0.25) (layer "B.Cu") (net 26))
 (segment (start 93.98 127) (end 93.98 128.1251) (width 0.25) (layer "B.Cu") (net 26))
 (segment (start 54.4651 142.0068) (end 54.4651 142.24) (width 0.25) (layer "F.Cu") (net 5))
 (segment (start 53.34 142.24) (end 54.4651 142.24) (width 0.25) (layer "F.Cu") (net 5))
 (segment (start 61.8519 134.62) (end 54.4651 142.0068) (width 0.25) (layer "F.Cu") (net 5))
 (segment (start 76.2 134.62) (end 61.8519 134.62) (width 0.25) (layer "F.Cu") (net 5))
 (segment (start 77.1389 135.7451) (end 77.6149 135.2691) (width 0.25) (layer "F.Cu") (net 6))
 (segment (start 57.0051 142.0068) (end 63.2668 135.7451) (width 0.25) (layer "F.Cu") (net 6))
 (segment (start 78.74 134.62) (end 77.6149 134.62) (width 0.25) (layer "F.Cu") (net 6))
 (segment (start 55.88 142.24) (end 57.0051 142.24) (width 0.25) (layer "F.Cu") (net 6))
 (segment (start 77.6149 135.2691) (end 77.6149 134.62) (width 0.25) (layer "F.Cu") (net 6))
 (segment (start 57.0051 142.24) (end 57.0051 142.0068) (width 0.25) (layer "F.Cu") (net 6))
 (segment (start 63.2668 135.7451) (end 77.1389 135.7451) (width 0.25) (layer "F.Cu") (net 6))
 (segment (start 81.28 134.62) (end 80.1549 134.62) (width 0.25) (layer "F.Cu") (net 7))
 (segment (start 80.1549 134.62) (end 80.1549 134.8577) (width 0.25) (layer "F.Cu") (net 7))
 (segment (start 65.3567 136.1952) (end 59.5451 142.0068) (width 0.25) (layer "F.Cu") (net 7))
 (segment (start 78.8174 136.1952) (end 65.3567 136.1952) (width 0.25) (layer "F.Cu") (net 7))
 (segment (start 80.1549 134.8577) (end 78.8174 136.1952) (width 0.25) (layer "F.Cu") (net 7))
 (segment (start 59.5451 142.0068) (end 59.5451 142.24) (width 0.25) (layer "F.Cu") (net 7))
 (segment (start 58.42 142.24) (end 59.5451 142.24) (width 0.25) (layer "F.Cu") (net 7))
 (segment (start 83.82 134.62) (end 82.6949 134.62) (width 0.25) (layer "F.Cu") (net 8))
 (segment (start 82.6949 134.9013) (end 80.9509 136.6453) (width 0.25) (layer "F.Cu") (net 8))
 (segment (start 80.9509 136.6453) (end 67.4466 136.6453) (width 0.25) (layer "F.Cu") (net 8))
 (segment (start 82.6949 134.62) (end 82.6949 134.9013) (width 0.25) (layer "F.Cu") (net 8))
 (segment (start 62.0851 142.0068) (end 62.0851 142.24) (width 0.25) (layer "F.Cu") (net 8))
 (segment (start 60.96 142.24) (end 62.0851 142.24) (width 0.25) (layer "F.Cu") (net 8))
 (segment (start 67.4466 136.6453) (end 62.0851 142.0068) (width 0.25) (layer "F.Cu") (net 8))
 (segment (start 85.2349 134.62) (end 85.2349 134.9013) (width 0.25) (layer "F.Cu") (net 9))
 (segment (start 86.36 134.62) (end 85.2349 134.62) (width 0.25) (layer "F.Cu") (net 9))
 (segment (start 63.5 142.24) (end 64.6251 142.24) (width 0.25) (layer "F.Cu") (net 9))
 (segment (start 64.6251 142.0068) (end 64.6251 142.24) (width 0.25) (layer "F.Cu") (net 9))
 (segment (start 85.2349 134.9013) (end 80.4985 139.6377) (width 0.25) (layer "F.Cu") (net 9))
 (segment (start 80.4985 139.6377) (end 66.9942 139.6377) (width 0.25) (layer "F.Cu") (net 9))
 (segment (start 66.9942 139.6377) (end 64.6251 142.0068) (width 0.25) (layer "F.Cu") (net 9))
 (segment (start 68.6033 140.5686) (end 67.1651 142.0068) (width 0.25) (layer "F.Cu") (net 10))
 (segment (start 66.04 142.24) (end 67.1651 142.24) (width 0.25) (layer "F.Cu") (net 10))
 (segment (start 82.1076 140.5686) (end 68.6033 140.5686) (width 0.25) (layer "F.Cu") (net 10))
 (segment (start 67.1651 142.0068) (end 67.1651 142.24) (width 0.25) (layer "F.Cu") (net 10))
 (segment (start 87.7749 134.9013) (end 82.1076 140.5686) (width 0.25) (layer "F.Cu") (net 10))
 (segment (start 88.9 134.62) (end 87.7749 134.62) (width 0.25) (layer "F.Cu") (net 10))
 (segment (start 87.7749 134.62) (end 87.7749 134.9013) (width 0.25) (layer "F.Cu") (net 10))
 (segment (start 69.7051 142.0068) (end 69.7051 142.24) (width 0.25) (layer "F.Cu") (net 11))
 (segment (start 90.3149 134.9013) (end 84.1974 141.0188) (width 0.25) (layer "F.Cu") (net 11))
 (segment (start 91.44 134.62) (end 90.3149 134.62) (width 0.25) (layer "F.Cu") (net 11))
 (segment (start 84.1974 141.0188) (end 70.6931 141.0188) (width 0.25) (layer "F.Cu") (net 11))
 (segment (start 70.6931 141.0188) (end 69.7051 142.0068) (width 0.25) (layer "F.Cu") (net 11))
 (segment (start 90.3149 134.62) (end 90.3149 134.9013) (width 0.25) (layer "F.Cu") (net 11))
 (segment (start 68.58 142.24) (end 69.7051 142.24) (width 0.25) (layer "F.Cu") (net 11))
 (segment (start 71.12 142.24) (end 72.2451 142.24) (width 0.25) (layer "B.Cu") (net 12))
 (segment (start 94.4507 143.4453) (end 73.4504 143.4453) (width 0.25) (layer "B.Cu") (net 12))
 (segment (start 95.1954 142.7006) (end 94.4507 143.4453) (width 0.25) (layer "B.Cu") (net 12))
 (segment (start 93.98 135.7451) (end 95.1954 136.9605) (width 0.25) (layer "B.Cu") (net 12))
 (segment (start 95.1954 136.9605) (end 95.1954 142.7006) (width 0.25) (layer "B.Cu") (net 12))
 (segment (start 93.98 134.62) (end 93.98 135.7451) (width 0.25) (layer "B.Cu") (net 12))
 (segment (start 73.4504 143.4453) (end 72.2451 142.24) (width 0.25) (layer "B.Cu") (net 12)))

